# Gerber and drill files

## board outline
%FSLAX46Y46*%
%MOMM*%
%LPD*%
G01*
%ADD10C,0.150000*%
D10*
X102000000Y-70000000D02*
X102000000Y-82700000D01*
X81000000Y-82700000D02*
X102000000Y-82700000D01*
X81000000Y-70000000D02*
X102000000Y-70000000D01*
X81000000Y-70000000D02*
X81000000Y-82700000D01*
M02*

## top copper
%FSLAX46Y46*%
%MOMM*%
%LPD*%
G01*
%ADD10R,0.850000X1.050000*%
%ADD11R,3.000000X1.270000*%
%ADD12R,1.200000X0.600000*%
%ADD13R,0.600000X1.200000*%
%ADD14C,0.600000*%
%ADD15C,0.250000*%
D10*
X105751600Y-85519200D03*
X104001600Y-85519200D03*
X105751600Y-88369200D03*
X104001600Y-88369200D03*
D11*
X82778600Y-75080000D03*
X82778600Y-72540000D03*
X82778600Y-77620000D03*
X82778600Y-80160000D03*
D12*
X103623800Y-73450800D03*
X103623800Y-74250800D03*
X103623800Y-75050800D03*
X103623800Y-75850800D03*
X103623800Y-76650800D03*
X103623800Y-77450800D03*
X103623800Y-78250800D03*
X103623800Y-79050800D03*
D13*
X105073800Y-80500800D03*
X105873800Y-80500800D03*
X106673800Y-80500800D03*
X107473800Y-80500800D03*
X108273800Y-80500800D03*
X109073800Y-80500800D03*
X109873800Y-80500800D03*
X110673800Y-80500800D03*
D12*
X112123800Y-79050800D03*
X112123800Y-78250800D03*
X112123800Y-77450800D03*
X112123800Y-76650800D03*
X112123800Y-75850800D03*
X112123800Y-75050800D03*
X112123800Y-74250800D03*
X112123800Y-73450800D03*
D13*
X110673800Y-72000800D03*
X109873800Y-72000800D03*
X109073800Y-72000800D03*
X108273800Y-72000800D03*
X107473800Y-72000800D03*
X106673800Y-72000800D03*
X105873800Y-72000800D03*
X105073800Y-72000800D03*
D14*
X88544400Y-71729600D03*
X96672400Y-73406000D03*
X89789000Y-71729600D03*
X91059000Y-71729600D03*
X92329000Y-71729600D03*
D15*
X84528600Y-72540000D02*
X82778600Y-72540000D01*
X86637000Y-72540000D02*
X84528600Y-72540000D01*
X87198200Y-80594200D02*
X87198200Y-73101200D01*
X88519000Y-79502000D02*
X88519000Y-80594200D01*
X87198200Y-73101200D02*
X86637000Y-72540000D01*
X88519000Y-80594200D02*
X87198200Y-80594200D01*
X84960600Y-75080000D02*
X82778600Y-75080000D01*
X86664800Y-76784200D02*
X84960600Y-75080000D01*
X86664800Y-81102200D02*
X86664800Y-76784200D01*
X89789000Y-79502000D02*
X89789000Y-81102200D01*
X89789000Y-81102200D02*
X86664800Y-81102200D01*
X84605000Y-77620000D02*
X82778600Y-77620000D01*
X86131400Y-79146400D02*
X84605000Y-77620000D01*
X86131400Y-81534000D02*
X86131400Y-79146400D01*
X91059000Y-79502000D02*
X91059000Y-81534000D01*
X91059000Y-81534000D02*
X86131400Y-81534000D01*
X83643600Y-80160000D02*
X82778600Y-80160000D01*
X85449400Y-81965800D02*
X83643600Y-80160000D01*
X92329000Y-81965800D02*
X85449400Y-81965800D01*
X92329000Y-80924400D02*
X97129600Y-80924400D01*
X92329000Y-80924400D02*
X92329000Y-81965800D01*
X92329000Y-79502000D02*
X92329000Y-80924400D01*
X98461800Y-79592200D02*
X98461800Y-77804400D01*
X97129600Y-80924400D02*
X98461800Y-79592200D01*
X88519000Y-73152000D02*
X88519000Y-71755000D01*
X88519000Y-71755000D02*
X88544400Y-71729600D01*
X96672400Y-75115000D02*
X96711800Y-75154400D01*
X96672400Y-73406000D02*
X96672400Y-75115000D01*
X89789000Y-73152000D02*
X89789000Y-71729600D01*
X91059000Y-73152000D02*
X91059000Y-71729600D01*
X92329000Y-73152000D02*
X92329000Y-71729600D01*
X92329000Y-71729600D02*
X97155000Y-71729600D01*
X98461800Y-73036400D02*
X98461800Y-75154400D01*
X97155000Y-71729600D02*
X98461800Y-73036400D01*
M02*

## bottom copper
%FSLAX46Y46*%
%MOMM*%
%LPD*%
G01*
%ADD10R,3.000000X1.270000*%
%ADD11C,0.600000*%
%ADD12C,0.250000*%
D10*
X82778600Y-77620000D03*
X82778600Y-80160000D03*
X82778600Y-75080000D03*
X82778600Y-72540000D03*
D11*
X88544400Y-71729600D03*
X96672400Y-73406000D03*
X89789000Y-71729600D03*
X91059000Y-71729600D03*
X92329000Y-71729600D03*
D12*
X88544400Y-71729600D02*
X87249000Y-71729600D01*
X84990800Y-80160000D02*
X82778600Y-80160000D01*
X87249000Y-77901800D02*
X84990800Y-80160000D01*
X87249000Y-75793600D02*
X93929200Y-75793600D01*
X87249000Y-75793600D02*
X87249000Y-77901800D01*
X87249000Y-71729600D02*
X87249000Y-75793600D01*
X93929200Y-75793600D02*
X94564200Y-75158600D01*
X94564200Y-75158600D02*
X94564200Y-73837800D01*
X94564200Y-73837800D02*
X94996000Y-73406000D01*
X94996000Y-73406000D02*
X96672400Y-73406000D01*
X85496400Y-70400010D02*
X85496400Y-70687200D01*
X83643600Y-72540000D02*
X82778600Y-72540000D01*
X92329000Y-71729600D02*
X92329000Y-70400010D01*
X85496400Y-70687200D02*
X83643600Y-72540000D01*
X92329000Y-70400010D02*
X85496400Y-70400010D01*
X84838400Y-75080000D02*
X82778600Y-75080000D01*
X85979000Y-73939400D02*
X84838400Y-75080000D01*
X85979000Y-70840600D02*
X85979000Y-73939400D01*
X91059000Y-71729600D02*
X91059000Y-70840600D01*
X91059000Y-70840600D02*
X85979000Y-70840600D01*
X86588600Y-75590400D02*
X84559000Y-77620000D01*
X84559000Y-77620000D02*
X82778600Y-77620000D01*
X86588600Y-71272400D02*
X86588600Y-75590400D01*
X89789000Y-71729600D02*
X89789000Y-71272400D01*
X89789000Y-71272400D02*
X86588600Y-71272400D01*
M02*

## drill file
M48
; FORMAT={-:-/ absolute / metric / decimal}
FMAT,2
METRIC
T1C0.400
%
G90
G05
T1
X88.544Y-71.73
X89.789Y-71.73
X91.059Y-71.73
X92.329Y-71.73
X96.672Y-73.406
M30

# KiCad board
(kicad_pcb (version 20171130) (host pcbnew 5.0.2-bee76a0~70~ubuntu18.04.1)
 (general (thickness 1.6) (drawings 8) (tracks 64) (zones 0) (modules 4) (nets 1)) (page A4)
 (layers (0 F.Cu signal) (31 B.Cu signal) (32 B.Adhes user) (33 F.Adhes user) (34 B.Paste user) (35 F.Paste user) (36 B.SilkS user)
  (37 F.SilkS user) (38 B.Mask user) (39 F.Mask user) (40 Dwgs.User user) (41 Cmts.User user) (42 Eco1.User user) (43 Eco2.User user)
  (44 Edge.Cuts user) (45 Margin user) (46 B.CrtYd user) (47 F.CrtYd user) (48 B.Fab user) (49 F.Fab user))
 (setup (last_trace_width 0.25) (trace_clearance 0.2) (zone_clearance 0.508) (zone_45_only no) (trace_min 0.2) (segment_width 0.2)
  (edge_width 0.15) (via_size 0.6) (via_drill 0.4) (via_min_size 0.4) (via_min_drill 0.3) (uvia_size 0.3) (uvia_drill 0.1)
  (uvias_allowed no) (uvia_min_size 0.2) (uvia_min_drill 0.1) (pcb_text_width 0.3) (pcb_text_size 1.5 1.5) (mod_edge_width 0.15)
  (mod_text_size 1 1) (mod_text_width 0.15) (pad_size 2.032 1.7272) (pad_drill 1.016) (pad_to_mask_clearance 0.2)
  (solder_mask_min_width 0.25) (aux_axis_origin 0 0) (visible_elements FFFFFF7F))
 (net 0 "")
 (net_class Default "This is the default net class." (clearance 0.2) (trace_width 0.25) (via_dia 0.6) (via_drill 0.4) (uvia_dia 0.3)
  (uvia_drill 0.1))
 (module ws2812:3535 (layer F.Cu) (at 104.8766 86.9442 90)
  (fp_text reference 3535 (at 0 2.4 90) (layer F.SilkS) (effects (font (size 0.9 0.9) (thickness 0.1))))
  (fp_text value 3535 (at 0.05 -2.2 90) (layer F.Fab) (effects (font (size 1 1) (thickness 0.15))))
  (pad IN smd rect (at 1.325 0.875 90) (size 1.05 0.85) (drill (offset 0.1 0)) (layers F.Cu F.Paste F.Mask))
  (pad VDD smd rect (at 1.325 -0.875 90) (size 1.05 0.85) (drill (offset 0.1 0)) (layers F.Cu F.Paste F.Mask))
  (pad GND smd rect (at -1.325 0.875 90) (size 1.05 0.85) (drill (offset -0.1 0)) (layers F.Cu F.Paste F.Mask))
  (pad OUT smd rect (at -1.325 -0.875 90) (size 1.05 0.85) (drill (offset -0.1 0)) (layers F.Cu F.Paste F.Mask)))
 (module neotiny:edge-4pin (layer F.Cu) (at 82.7786 80.16 90)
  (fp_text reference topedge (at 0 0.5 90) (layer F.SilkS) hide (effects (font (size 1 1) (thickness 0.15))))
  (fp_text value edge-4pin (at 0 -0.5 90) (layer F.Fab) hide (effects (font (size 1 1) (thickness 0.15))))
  (pad 3 connect rect (at 5.08 0 90) (size 1.27 3) (layers F.Cu F.Mask))
  (pad 4 connect rect (at 7.62 0 90) (size 1.27 3) (layers F.Cu F.Mask))
  (pad 2 connect rect (at 2.54 0 90) (size 1.27 3) (layers F.Cu F.Mask))
  (pad 1 connect rect (at 0 0 90) (size 1.27 3) (layers F.Cu F.Mask)))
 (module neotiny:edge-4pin (layer B.Cu) (at 82.7786 72.54 270)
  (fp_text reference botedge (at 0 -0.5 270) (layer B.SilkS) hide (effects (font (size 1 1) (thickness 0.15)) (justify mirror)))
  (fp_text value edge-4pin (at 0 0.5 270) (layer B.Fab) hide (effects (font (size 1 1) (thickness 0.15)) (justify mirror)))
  (pad 3 connect rect (at 5.08 0 270) (size 1.27 3) (layers B.Cu B.Mask))
  (pad 4 connect rect (at 7.62 0 270) (size 1.27 3) (layers B.Cu B.Mask))
  (pad 2 connect rect (at 2.54 0 270) (size 1.27 3) (layers B.Cu B.Mask))
  (pad 1 connect rect (at 0 0 270) (size 1.27 3) (layers B.Cu B.Mask)))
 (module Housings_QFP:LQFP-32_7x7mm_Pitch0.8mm (layer F.Cu) (at 107.8738 76.2508)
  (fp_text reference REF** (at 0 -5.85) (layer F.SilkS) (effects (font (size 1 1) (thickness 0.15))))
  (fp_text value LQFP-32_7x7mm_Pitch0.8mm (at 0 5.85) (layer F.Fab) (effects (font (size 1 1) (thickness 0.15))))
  (pad 1 smd rect (at -4.25 -2.8) (size 1.2 0.6) (layers F.Cu F.Paste F.Mask))
  (pad 2 smd rect (at -4.25 -2) (size 1.2 0.6) (layers F.Cu F.Paste F.Mask))
  (pad 3 smd rect (at -4.25 -1.2) (size 1.2 0.6) (layers F.Cu F.Paste F.Mask))
  (pad 4 smd rect (at -4.25 -0.4) (size 1.2 0.6) (layers F.Cu F.Paste F.Mask))
  (pad 5 smd rect (at -4.25 0.4) (size 1.2 0.6) (layers F.Cu F.Paste F.Mask))
  (pad 6 smd rect (at -4.25 1.2) (size 1.2 0.6) (layers F.Cu F.Paste F.Mask))
  (pad 7 smd rect (at -4.25 2) (size 1.2 0.6) (layers F.Cu F.Paste F.Mask))
  (pad 8 smd rect (at -4.25 2.8) (size 1.2 0.6) (layers F.Cu F.Paste F.Mask))
  (pad 9 smd rect (at -2.8 4.25 90) (size 1.2 0.6) (layers F.Cu F.Paste F.Mask))
  (pad 10 smd rect (at -2 4.25 90) (size 1.2 0.6) (layers F.Cu F.Paste F.Mask))
  (pad 11 smd rect (at -1.2 4.25 90) (size 1.2 0.6) (layers F.Cu F.Paste F.Mask))
  (pad 12 smd rect (at -0.4 4.25 90) (size 1.2 0.6) (layers F.Cu F.Paste F.Mask))
  (pad 13 smd rect (at 0.4 4.25 90) (size 1.2 0.6) (layers F.Cu F.Paste F.Mask))
  (pad 14 smd rect (at 1.2 4.25 90) (size 1.2 0.6) (layers F.Cu F.Paste F.Mask))
  (pad 15 smd rect (at 2 4.25 90) (size 1.2 0.6) (layers F.Cu F.Paste F.Mask))
  (pad 16 smd rect (at 2.8 4.25 90) (size 1.2 0.6) (layers F.Cu F.Paste F.Mask))
  (pad 17 smd rect (at 4.25 2.8) (size 1.2 0.6) (layers F.Cu F.Paste F.Mask))
  (pad 18 smd rect (at 4.25 2) (size 1.2 0.6) (layers F.Cu F.Paste F.Mask))
  (pad 19 smd rect (at 4.25 1.2) (size 1.2 0.6) (layers F.Cu F.Paste F.Mask))
  (pad 20 smd rect (at 4.25 0.4) (size 1.2 0.6) (layers F.Cu F.Paste F.Mask))
  (pad 21 smd rect (at 4.25 -0.4) (size 1.2 0.6) (layers F.Cu F.Paste F.Mask))
  (pad 22 smd rect (at 4.25 -1.2) (size 1.2 0.6) (layers F.Cu F.Paste F.Mask))
  (pad 23 smd rect (at 4.25 -2) (size 1.2 0.6) (layers F.Cu F.Paste F.Mask))
  (pad 24 smd rect (at 4.25 -2.8) (size 1.2 0.6) (layers F.Cu F.Paste F.Mask))
  (pad 25 smd rect (at 2.8 -4.25 90) (size 1.2 0.6) (layers F.Cu F.Paste F.Mask))
  (pad 26 smd rect (at 2 -4.25 90) (size 1.2 0.6) (layers F.Cu F.Paste F.Mask))
  (pad 27 smd rect (at 1.2 -4.25 90) (size 1.2 0.6) (layers F.Cu F.Paste F.Mask))
  (pad 28 smd rect (at 0.4 -4.25 90) (size 1.2 0.6) (layers F.Cu F.Paste F.Mask))
  (pad 29 smd rect (at -0.4 -4.25 90) (size 1.2 0.6) (layers F.Cu F.Paste F.Mask))
  (pad 30 smd rect (at -1.2 -4.25 90) (size 1.2 0.6) (layers F.Cu F.Paste F.Mask))
  (pad 31 smd rect (at -2 -4.25 90) (size 1.2 0.6) (layers F.Cu F.Paste F.Mask))
  (pad 32 smd rect (at -2.8 -4.25 90) (size 1.2 0.6) (layers F.Cu F.Paste F.Mask)))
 (gr_line (start 102 70) (end 102 82.7) (angle 90) (layer Edge.Cuts) (width 0.15))
 (gr_line (start 81 82.7) (end 102 82.7) (angle 90) (layer Edge.Cuts) (width 0.15))
 (gr_line (start 81 70) (end 102 70) (angle 90) (layer Edge.Cuts) (width 0.15))
 (gr_line (start 81 70) (end 81 82.7) (angle 90) (layer Edge.Cuts) (width 0.15))
 (segment (start 84.5286 72.54) (end 82.7786 72.54) (width 0.25) (layer F.Cu) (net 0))
 (segment (start 86.637 72.54) (end 84.5286 72.54) (width 0.25) (layer F.Cu) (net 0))
 (segment (start 87.1982 80.5942) (end 87.1982 73.1012) (width 0.25) (layer F.Cu) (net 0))
 (segment (start 88.519 79.502) (end 88.519 80.5942) (width 0.25) (layer F.Cu) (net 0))
 (segment (start 87.1982 73.1012) (end 86.637 72.54) (width 0.25) (layer F.Cu) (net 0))
 (segment (start 88.519 80.5942) (end 87.1982 80.5942) (width 0.25) (layer F.Cu) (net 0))
 (segment (start 84.9606 75.08) (end 82.7786 75.08) (width 0.25) (layer F.Cu) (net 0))
 (segment (start 86.6648 76.7842) (end 84.9606 75.08) (width 0.25) (layer F.Cu) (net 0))
 (segment (start 86.6648 81.1022) (end 86.6648 76.7842) (width 0.25) (layer F.Cu) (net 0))
 (segment (start 89.789 79.502) (end 89.789 81.1022) (width 0.25) (layer F.Cu) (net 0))
 (segment (start 89.789 81.1022) (end 86.6648 81.1022) (width 0.25) (layer F.Cu) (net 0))
 (segment (start 84.605 77.62) (end 82.7786 77.62) (width 0.25) (layer F.Cu) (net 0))
 (segment (start 86.1314 79.1464) (end 84.605 77.62) (width 0.25) (layer F.Cu) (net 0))
 (segment (start 86.1314 81.534) (end 86.1314 79.1464) (width 0.25) (layer F.Cu) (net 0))
 (segment (start 91.059 79.502) (end 91.059 81.534) (width 0.25) (layer F.Cu) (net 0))
 (segment (start 91.059 81.534) (end 86.1314 81.534) (width 0.25) (layer F.Cu) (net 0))
 (segment (start 83.6436 80.16) (end 82.7786 80.16) (width 0.25) (layer F.Cu) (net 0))
 (segment (start 85.4494 81.9658) (end 83.6436 80.16) (width 0.25) (layer F.Cu) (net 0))
 (segment (start 92.329 81.9658) (end 85.4494 81.9658) (width 0.25) (layer F.Cu) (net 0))
 (segment (start 92.329 80.9244) (end 97.1296 80.9244) (width 0.25) (layer F.Cu) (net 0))
 (segment (start 92.329 80.9244) (end 92.329 81.9658) (width 0.25) (layer F.Cu) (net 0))
 (segment (start 92.329 79.502) (end 92.329 80.9244) (width 0.25) (layer F.Cu) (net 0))
 (segment (start 98.4618 79.5922) (end 98.4618 77.8044) (width 0.25) (layer F.Cu) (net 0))
 (segment (start 97.1296 80.9244) (end 98.4618 79.5922) (width 0.25) (layer F.Cu) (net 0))
 (via (at 88.5444 71.7296) (size 0.6) (drill 0.4) (layers F.Cu B.Cu) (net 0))
 (segment (start 88.519 73.152) (end 88.519 71.755) (width 0.25) (layer F.Cu) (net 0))
 (segment (start 88.519 71.755) (end 88.5444 71.7296) (width 0.25) (layer F.Cu) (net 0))
 (segment (start 88.5444 71.7296) (end 87.249 71.7296) (width 0.25) (layer B.Cu) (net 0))
 (segment (start 84.9908 80.16) (end 82.7786 80.16) (width 0.25) (layer B.Cu) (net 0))
 (segment (start 87.249 77.9018) (end 84.9908 80.16) (width 0.25) (layer B.Cu) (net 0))
 (segment (start 87.249 75.7936) (end 93.9292 75.7936) (width 0.25) (layer B.Cu) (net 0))
 (segment (start 87.249 75.7936) (end 87.249 77.9018) (width 0.25) (layer B.Cu) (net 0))
 (segment (start 87.249 71.7296) (end 87.249 75.7936) (width 0.25) (layer B.Cu) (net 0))
 (segment (start 93.9292 75.7936) (end 94.5642 75.1586) (width 0.25) (layer B.Cu) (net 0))
 (segment (start 94.5642 75.1586) (end 94.5642 73.8378) (width 0.25) (layer B.Cu) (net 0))
 (segment (start 94.5642 73.8378) (end 94.996 73.406) (width 0.25) (layer B.Cu) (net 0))
 (via (at 96.6724 73.406) (size 0.6) (drill 0.4) (layers F.Cu B.Cu) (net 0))
 (segment (start 94.996 73.406) (end 96.6724 73.406) (width 0.25) (layer B.Cu) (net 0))
 (segment (start 96.6724 75.115) (end 96.7118 75.1544) (width 0.25) (layer F.Cu) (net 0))
 (segment (start 96.6724 73.406) (end 96.6724 75.115) (width 0.25) (layer F.Cu) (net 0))
 (via (at 89.789 71.7296) (size 0.6) (drill 0.4) (layers F.Cu B.Cu) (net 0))
 (segment (start 89.789 73.152) (end 89.789 71.7296) (width 0.25) (layer F.Cu) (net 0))
 (via (at 91.059 71.7296) (size 0.6) (drill 0.4) (layers F.Cu B.Cu) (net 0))
 (segment (start 91.059 73.152) (end 91.059 71.7296) (width 0.25) (layer F.Cu) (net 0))
 (via (at 92.329 71.7296) (size 0.6) (drill 0.4) (layers F.Cu B.Cu) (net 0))
 (segment (start 92.329 73.152) (end 92.329 71.7296) (width 0.25) (layer F.Cu) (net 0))
 (segment (start 85.4964 70.40001) (end 85.4964 70.6872) (width 0.25) (layer B.Cu) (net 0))
 (segment (start 83.6436 72.54) (end 82.7786 72.54) (width 0.25) (layer B.Cu) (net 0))
 (segment (start 92.329 71.7296) (end 92.329 70.40001) (width 0.25) (layer B.Cu) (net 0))
 (segment (start 85.4964 70.6872) (end 83.6436 72.54) (width 0.25) (layer B.Cu) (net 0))
 (segment (start 92.329 70.40001) (end 85.4964 70.40001) (width 0.25) (layer B.Cu) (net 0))
 (segment (start 84.8384 75.08) (end 82.7786 75.08) (width 0.25) (layer B.Cu) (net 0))
 (segment (start 85.979 73.9394) (end 84.8384 75.08) (width 0.25) (layer B.Cu) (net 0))
 (segment (start 85.979 70.8406) (end 85.979 73.9394) (width 0.25) (layer B.Cu) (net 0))
 (segment (start 91.059 71.7296) (end 91.059 70.8406) (width 0.25) (layer B.Cu) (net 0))
 (segment (start 91.059 70.8406) (end 85.979 70.8406) (width 0.25) (layer B.Cu) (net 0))
 (segment (start 86.5886 75.5904) (end 84.559 77.62) (width 0.25) (layer B.Cu) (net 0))
 (segment (start 84.559 77.62) (end 82.7786 77.62) (width 0.25) (layer B.Cu) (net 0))
 (segment (start 86.5886 71.2724) (end 86.5886 75.5904) (width 0.25) (layer B.Cu) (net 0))
 (segment (start 89.789 71.7296) (end 89.789 71.2724) (width 0.25) (layer B.Cu) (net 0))
 (segment (start 89.789 71.2724) (end 86.5886 71.2724) (width 0.25) (layer B.Cu) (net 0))
 (segment (start 92.329 71.7296) (end 97.155 71.7296) (width 0.25) (layer F.Cu) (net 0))
 (segment (start 98.4618 73.0364) (end 98.4618 75.1544) (width 0.25) (layer F.Cu) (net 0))
 (segment (start 97.155 71.7296) (end 98.4618 73.0364) (width 0.25) (layer F.Cu) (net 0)))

